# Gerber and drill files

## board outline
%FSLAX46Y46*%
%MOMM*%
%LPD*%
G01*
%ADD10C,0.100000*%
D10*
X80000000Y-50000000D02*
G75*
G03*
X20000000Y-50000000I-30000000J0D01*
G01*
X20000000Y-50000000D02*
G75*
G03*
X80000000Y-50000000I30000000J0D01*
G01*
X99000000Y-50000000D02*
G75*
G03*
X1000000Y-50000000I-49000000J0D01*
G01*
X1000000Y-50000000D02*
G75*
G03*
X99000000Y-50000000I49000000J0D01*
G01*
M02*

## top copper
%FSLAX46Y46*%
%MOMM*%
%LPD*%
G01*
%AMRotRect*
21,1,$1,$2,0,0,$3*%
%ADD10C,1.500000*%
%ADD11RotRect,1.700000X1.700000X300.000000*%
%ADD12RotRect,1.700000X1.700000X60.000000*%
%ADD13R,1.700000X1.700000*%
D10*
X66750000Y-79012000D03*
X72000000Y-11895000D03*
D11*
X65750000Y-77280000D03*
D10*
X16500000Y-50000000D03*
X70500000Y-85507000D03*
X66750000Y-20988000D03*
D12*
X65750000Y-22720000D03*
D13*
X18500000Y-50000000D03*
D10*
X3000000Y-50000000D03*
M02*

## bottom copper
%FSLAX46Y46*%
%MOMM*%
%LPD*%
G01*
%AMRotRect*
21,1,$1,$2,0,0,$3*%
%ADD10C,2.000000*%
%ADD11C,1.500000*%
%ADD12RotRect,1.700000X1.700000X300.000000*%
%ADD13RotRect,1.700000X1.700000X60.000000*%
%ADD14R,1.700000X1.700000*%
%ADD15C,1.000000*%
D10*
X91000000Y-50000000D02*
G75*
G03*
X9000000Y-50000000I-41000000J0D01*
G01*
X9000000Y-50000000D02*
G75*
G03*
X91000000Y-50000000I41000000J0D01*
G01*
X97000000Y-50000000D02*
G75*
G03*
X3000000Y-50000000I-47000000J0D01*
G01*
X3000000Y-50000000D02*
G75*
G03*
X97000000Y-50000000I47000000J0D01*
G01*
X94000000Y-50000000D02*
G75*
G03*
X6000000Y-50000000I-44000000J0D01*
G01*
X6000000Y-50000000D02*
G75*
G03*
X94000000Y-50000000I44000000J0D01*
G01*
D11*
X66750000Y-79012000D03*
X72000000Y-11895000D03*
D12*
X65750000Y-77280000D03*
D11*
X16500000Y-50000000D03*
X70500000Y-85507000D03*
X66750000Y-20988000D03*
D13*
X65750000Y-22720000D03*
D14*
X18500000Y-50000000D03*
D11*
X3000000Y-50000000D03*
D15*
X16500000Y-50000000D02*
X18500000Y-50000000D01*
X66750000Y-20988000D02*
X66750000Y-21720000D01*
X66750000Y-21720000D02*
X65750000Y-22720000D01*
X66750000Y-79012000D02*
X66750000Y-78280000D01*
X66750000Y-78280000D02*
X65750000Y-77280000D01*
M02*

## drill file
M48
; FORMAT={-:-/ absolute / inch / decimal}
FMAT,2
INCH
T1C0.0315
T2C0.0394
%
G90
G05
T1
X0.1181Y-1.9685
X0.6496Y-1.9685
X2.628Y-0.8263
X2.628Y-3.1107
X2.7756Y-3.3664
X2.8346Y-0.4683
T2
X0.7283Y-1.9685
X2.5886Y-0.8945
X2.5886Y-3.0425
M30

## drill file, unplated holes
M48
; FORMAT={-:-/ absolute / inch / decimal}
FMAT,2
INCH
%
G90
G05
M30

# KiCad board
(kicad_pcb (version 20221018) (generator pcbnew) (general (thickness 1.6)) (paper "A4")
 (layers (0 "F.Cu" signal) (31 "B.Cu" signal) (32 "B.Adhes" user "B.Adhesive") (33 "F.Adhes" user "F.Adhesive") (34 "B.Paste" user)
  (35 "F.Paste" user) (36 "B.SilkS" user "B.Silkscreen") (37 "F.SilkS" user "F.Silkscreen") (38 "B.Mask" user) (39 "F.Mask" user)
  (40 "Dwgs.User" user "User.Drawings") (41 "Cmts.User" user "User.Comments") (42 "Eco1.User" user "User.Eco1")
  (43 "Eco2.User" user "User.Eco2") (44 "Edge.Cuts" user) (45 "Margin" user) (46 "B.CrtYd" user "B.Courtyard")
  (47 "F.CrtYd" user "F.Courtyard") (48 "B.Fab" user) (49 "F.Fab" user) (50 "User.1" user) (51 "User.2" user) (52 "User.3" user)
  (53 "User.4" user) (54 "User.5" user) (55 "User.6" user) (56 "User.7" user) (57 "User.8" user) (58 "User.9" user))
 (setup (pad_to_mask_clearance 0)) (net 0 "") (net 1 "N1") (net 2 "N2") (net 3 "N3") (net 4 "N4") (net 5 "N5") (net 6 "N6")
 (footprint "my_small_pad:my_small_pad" (layer "F.Cu") (at 66.75 79.012)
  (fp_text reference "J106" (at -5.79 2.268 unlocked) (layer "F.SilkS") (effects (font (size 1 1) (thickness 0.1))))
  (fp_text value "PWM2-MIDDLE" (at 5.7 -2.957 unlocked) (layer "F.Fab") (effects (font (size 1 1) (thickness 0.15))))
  (pad "1" thru_hole circle (at 0 0) (size 1.5 1.5) (drill 0.8) (layers "*.Cu" "*.Mask") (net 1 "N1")))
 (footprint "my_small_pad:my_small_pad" (layer "F.Cu") (at 72 11.895)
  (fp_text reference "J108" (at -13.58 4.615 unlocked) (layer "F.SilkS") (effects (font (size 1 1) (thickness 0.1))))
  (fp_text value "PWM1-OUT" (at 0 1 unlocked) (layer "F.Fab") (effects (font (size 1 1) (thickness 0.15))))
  (pad "1" thru_hole circle (at 0 0) (size 1.5 1.5) (drill 0.8) (layers "*.Cu" "*.Mask") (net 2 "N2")))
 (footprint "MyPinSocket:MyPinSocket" (layer "F.Cu") (at 65.75 77.28 -60)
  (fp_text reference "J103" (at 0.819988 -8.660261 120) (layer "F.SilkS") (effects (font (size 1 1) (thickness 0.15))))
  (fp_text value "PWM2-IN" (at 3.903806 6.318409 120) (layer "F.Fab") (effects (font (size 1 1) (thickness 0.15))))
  (pad "1" thru_hole rect (at 0 0 300) (size 1.7 1.7) (drill 1) (layers "*.Cu" "*.Mask") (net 1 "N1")))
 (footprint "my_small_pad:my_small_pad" (layer "F.Cu") (at 16.5 50)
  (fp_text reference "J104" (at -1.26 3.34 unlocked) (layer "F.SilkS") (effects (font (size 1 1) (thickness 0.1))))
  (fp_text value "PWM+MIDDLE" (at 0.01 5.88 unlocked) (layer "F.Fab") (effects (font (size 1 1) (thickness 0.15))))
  (pad "1" thru_hole circle (at 0 0) (size 1.5 1.5) (drill 0.8) (layers "*.Cu" "*.Mask") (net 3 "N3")))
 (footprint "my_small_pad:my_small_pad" (layer "F.Cu") (at 70.5 85.507)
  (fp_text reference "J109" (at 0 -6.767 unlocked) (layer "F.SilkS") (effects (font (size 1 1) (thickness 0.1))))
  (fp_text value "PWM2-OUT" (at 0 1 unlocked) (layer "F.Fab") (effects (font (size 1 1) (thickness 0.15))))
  (pad "1" thru_hole circle (at 0 0) (size 1.5 1.5) (drill 0.8) (layers "*.Cu" "*.Mask") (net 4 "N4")))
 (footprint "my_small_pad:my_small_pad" (layer "F.Cu") (at 66.75 20.988)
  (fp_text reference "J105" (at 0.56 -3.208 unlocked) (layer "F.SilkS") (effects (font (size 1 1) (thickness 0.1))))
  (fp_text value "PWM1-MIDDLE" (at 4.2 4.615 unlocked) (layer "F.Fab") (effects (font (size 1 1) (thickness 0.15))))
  (pad "1" thru_hole circle (at 0 0) (size 1.5 1.5) (drill 0.8) (layers "*.Cu" "*.Mask") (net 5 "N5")))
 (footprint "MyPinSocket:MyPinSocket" (layer "F.Cu") (at 65.75 22.72 60)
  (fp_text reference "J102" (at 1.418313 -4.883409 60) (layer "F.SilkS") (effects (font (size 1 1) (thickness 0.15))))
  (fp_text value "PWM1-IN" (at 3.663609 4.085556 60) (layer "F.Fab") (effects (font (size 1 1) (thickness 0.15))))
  (pad "1" thru_hole rect (at 0 0 60) (size 1.7 1.7) (drill 1) (layers "*.Cu" "*.Mask") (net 5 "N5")))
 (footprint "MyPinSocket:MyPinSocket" (layer "F.Cu") (at 18.5 50)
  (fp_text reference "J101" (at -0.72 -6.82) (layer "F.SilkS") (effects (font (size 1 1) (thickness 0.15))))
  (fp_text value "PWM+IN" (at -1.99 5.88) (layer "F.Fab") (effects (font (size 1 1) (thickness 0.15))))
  (pad "1" thru_hole rect (at 0 0) (size 1.7 1.7) (drill 1) (layers "*.Cu" "*.Mask") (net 3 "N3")))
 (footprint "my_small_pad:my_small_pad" (layer "F.Cu") (at 3 50)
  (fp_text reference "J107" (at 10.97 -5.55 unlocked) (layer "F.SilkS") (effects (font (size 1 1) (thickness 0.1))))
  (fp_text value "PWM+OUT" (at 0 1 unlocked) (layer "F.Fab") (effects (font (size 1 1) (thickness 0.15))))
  (pad "1" thru_hole circle (at 0 0) (size 1.5 1.5) (drill 0.8) (layers "*.Cu" "*.Mask") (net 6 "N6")))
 (gr_circle (center 50 50) (end 91 50) (stroke (width 2) (type default)) (fill none) (layer "B.Cu"))
 (gr_circle (center 50 50) (end 97 50) (stroke (width 2) (type default)) (fill none) (layer "B.Cu"))
 (gr_circle (center 50 50) (end 94 50) (stroke (width 2) (type default)) (fill none) (layer "B.Cu"))
 (gr_circle (center 50 50) (end 80 50) (stroke (width 0.1) (type default)) (fill none) (layer "Edge.Cuts"))
 (gr_circle (center 50 50) (end 99 50) (stroke (width 0.1) (type default)) (fill none) (layer "Edge.Cuts"))
 (segment (start 16.5 50) (end 18.5 50) (width 1) (layer "B.Cu") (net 3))
 (segment (start 66.75 20.988) (end 66.75 21.72) (width 1) (layer "B.Cu") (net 5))
 (segment (start 66.75 21.72) (end 65.75 22.72) (width 1) (layer "B.Cu") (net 5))
 (segment (start 66.75 79.012) (end 66.75 78.28) (width 1) (layer "B.Cu") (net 1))
 (segment (start 66.75 78.28) (end 65.75 77.28) (width 1) (layer "B.Cu") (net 1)))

